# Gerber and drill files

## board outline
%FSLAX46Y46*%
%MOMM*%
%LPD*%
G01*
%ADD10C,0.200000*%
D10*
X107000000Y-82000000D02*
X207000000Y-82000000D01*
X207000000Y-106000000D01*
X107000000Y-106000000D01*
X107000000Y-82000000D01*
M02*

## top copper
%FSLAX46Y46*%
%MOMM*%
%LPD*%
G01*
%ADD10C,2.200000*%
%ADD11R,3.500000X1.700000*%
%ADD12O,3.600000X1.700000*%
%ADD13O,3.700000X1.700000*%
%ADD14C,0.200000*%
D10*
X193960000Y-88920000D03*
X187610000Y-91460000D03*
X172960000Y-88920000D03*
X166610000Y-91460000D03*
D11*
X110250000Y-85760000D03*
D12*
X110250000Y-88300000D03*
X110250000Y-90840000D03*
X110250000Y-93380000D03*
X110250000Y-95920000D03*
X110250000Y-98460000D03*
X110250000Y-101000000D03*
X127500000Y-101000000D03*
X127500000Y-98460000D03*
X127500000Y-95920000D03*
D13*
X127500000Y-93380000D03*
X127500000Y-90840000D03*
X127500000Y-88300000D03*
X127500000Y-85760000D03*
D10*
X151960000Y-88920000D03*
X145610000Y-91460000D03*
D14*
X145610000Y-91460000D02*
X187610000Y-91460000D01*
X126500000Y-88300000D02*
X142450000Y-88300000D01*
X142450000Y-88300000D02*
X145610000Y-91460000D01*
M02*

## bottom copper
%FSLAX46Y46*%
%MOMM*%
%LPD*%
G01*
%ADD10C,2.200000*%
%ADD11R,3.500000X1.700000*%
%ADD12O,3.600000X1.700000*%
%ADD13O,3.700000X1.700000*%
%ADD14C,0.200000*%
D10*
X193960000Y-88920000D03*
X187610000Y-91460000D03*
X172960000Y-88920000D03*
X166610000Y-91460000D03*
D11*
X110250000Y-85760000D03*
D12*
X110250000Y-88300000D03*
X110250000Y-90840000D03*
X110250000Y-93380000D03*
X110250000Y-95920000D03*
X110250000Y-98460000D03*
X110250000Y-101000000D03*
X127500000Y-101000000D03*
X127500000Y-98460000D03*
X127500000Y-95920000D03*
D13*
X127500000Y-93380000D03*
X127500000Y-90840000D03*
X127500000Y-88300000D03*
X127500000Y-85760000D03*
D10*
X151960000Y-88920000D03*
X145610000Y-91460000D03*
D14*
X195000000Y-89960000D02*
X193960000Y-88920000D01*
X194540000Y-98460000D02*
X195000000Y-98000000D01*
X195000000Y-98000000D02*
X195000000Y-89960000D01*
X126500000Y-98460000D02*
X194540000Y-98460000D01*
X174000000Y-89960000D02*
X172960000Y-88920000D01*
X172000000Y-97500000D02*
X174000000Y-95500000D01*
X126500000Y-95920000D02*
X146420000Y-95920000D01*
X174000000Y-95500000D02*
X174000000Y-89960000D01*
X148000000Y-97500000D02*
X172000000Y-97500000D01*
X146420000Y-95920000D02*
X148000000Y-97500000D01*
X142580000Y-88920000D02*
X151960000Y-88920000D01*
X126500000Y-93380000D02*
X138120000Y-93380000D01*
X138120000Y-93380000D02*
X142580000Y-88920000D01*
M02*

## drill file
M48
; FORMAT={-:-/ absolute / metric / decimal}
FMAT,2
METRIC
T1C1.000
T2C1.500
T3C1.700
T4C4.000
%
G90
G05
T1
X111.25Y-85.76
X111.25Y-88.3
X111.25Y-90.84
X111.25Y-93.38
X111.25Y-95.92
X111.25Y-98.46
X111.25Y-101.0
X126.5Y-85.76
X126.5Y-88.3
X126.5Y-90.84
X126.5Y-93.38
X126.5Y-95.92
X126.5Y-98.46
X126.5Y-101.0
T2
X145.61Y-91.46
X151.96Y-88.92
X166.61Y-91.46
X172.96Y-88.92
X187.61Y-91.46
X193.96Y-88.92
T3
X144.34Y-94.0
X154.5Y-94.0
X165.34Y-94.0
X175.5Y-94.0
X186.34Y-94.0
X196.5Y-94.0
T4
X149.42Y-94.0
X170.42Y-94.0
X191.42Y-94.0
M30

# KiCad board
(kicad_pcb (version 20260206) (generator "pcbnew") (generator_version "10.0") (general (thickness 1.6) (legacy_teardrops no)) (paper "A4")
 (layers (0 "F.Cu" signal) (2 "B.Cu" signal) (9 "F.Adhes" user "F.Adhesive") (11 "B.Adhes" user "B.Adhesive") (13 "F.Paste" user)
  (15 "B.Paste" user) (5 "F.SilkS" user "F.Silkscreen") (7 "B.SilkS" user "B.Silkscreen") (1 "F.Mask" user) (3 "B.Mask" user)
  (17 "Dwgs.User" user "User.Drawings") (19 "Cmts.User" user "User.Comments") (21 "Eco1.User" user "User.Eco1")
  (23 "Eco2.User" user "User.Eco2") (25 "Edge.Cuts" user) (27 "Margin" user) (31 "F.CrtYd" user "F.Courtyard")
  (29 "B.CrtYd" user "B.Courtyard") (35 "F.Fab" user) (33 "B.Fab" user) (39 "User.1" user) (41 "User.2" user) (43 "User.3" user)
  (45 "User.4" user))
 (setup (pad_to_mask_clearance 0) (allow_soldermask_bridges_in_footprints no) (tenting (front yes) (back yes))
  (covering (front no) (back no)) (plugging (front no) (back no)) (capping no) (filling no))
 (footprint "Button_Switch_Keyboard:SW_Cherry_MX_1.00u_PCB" (layer "F.Cu") (at 193.96 88.92)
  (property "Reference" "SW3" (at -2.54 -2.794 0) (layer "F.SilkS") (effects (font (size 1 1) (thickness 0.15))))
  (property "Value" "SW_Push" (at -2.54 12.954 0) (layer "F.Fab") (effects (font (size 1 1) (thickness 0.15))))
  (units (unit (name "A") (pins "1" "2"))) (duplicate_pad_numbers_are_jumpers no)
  (pad "" np_thru_hole circle (at -7.62 5.08) (size 1.7 1.7) (drill 1.7) (layers "*.Cu" "*.Mask"))
  (pad "" np_thru_hole circle (at -2.54 5.08) (size 4 4) (drill 4) (layers "*.Cu" "*.Mask"))
  (pad "" np_thru_hole circle (at 2.54 5.08) (size 1.7 1.7) (drill 1.7) (layers "*.Cu" "*.Mask"))
  (pad "1" thru_hole circle (at 0 0) (size 2.2 2.2) (drill 1.5) (layers "*.Cu" "*.Mask") (remove_unused_layers no)
   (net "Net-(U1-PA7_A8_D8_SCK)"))
  (pad "2" thru_hole circle (at -6.35 2.54) (size 2.2 2.2) (drill 1.5) (layers "*.Cu" "*.Mask") (remove_unused_layers no) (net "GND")))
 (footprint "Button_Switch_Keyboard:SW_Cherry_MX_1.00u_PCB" (layer "F.Cu") (at 172.96 88.92)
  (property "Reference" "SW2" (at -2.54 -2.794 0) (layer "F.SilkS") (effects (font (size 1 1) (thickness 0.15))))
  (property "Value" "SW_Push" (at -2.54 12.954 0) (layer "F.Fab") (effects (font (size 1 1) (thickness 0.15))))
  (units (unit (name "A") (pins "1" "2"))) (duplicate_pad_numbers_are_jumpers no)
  (pad "" np_thru_hole circle (at -7.62 5.08) (size 1.7 1.7) (drill 1.7) (layers "*.Cu" "*.Mask"))
  (pad "" np_thru_hole circle (at -2.54 5.08) (size 4 4) (drill 4) (layers "*.Cu" "*.Mask"))
  (pad "" np_thru_hole circle (at 2.54 5.08) (size 1.7 1.7) (drill 1.7) (layers "*.Cu" "*.Mask"))
  (pad "1" thru_hole circle (at 0 0) (size 2.2 2.2) (drill 1.5) (layers "*.Cu" "*.Mask") (remove_unused_layers no)
   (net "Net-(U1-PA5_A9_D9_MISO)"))
  (pad "2" thru_hole circle (at -6.35 2.54) (size 2.2 2.2) (drill 1.5) (layers "*.Cu" "*.Mask") (remove_unused_layers no) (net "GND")))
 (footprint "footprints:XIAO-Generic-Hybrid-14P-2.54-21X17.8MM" (layer "F.Cu") (at 118.875 93.38)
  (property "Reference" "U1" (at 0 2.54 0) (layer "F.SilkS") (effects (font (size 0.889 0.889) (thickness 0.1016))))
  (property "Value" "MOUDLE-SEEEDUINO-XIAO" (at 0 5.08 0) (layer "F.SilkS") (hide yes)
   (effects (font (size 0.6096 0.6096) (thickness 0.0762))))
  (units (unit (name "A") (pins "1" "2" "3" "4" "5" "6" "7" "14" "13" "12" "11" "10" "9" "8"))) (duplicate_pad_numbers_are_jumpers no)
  (pad "1" thru_hole rect (at -7.625 -7.62) (size 3.5 1.7) (drill 1 (offset -1 0)) (layers "*.Cu" "*.Mask") (remove_unused_layers no)
   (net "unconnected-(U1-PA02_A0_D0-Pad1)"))
  (pad "2" thru_hole oval (at -7.625 -5.08) (size 3.6 1.7) (drill 1 (offset -1 0)) (layers "*.Cu" "*.Mask") (remove_unused_layers no)
   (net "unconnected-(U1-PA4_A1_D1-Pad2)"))
  (pad "3" thru_hole oval (at -7.625 -2.54) (size 3.6 1.7) (drill 1 (offset -1 0)) (layers "*.Cu" "*.Mask") (remove_unused_layers no)
   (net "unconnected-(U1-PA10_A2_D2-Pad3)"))
  (pad "4" thru_hole oval (at -7.625 0) (size 3.6 1.7) (drill 1 (offset -1 0)) (layers "*.Cu" "*.Mask") (remove_unused_layers no)
   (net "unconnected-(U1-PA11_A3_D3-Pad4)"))
  (pad "5" thru_hole oval (at -7.625 2.54) (size 3.6 1.7) (drill 1 (offset -1 0)) (layers "*.Cu" "*.Mask") (remove_unused_layers no)
   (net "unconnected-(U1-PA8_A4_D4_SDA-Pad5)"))
  (pad "6" thru_hole oval (at -7.625 5.08 180) (size 3.6 1.7) (drill 1 (offset 1 0)) (layers "*.Cu" "*.Mask") (remove_unused_layers no)
   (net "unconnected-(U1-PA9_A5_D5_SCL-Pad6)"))
  (pad "7" thru_hole oval (at -7.625 7.62) (size 3.6 1.7) (drill 1 (offset -1 0)) (layers "*.Cu" "*.Mask") (remove_unused_layers no)
   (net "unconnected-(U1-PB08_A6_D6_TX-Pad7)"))
  (pad "8" thru_hole oval (at 7.625 7.62) (size 3.6 1.7) (drill 1 (offset 1 0)) (layers "*.Cu" "*.Mask") (remove_unused_layers no)
   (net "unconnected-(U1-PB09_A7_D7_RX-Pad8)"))
  (pad "9" thru_hole oval (at 7.625 5.08) (size 3.6 1.7) (drill 1 (offset 1 0)) (layers "*.Cu" "*.Mask") (remove_unused_layers no)
   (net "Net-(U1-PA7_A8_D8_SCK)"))
  (pad "10" thru_hole oval (at 7.625 2.54) (size 3.6 1.7) (drill 1 (offset 1 0)) (layers "*.Cu" "*.Mask") (remove_unused_layers no)
   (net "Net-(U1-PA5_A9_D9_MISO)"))
  (pad "11" thru_hole oval (at 7.625 0) (size 3.7 1.7) (drill 1 (offset 1 0)) (layers "*.Cu" "*.Mask") (remove_unused_layers no)
   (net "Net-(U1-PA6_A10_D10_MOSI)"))
  (pad "12" thru_hole oval (at 7.625 -2.54) (size 3.7 1.7) (drill 1 (offset 1 0)) (layers "*.Cu" "*.Mask") (remove_unused_layers no)
   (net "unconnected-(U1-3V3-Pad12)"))
  (pad "13" thru_hole oval (at 7.625 -5.08) (size 3.7 1.7) (drill 1 (offset 1 0)) (layers "*.Cu" "*.Mask") (remove_unused_layers no)
   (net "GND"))
  (pad "14" thru_hole oval (at 7.625 -7.62) (size 3.7 1.7) (drill 1 (offset 1 0)) (layers "*.Cu" "*.Mask") (remove_unused_layers no)
   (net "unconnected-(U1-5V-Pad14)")))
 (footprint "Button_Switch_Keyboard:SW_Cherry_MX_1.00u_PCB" (layer "F.Cu") (at 151.96 88.92)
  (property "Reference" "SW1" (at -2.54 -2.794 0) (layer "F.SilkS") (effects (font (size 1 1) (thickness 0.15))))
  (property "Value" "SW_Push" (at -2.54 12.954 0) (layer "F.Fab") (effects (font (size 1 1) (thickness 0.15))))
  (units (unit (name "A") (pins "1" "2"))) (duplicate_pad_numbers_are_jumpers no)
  (pad "" np_thru_hole circle (at -7.62 5.08) (size 1.7 1.7) (drill 1.7) (layers "*.Cu" "*.Mask"))
  (pad "" np_thru_hole circle (at -2.54 5.08) (size 4 4) (drill 4) (layers "*.Cu" "*.Mask"))
  (pad "" np_thru_hole circle (at 2.54 5.08) (size 1.7 1.7) (drill 1.7) (layers "*.Cu" "*.Mask"))
  (pad "1" thru_hole circle (at 0 0) (size 2.2 2.2) (drill 1.5) (layers "*.Cu" "*.Mask") (remove_unused_layers no)
   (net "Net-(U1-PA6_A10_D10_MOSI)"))
  (pad "2" thru_hole circle (at -6.35 2.54) (size 2.2 2.2) (drill 1.5) (layers "*.Cu" "*.Mask") (remove_unused_layers no) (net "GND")))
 (gr_rect (start 107 82) (end 207 106) (stroke (width 0.2) (type default)) (fill no) (layer "Edge.Cuts"))
 (segment (start 195 89.96) (end 193.96 88.92) (width 0.2) (layer "B.Cu") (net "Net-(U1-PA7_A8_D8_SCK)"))
 (segment (start 194.54 98.46) (end 195 98) (width 0.2) (layer "B.Cu") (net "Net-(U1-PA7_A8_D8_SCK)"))
 (segment (start 195 98) (end 195 89.96) (width 0.2) (layer "B.Cu") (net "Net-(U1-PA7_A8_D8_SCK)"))
 (segment (start 126.5 98.46) (end 194.54 98.46) (width 0.2) (layer "B.Cu") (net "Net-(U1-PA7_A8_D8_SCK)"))
 (segment (start 145.61 91.46) (end 187.61 91.46) (width 0.2) (layer "F.Cu") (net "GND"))
 (segment (start 126.5 88.3) (end 142.45 88.3) (width 0.2) (layer "F.Cu") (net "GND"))
 (segment (start 142.45 88.3) (end 145.61 91.46) (width 0.2) (layer "F.Cu") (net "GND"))
 (segment (start 174 89.96) (end 172.96 88.92) (width 0.2) (layer "B.Cu") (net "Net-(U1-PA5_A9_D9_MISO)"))
 (segment (start 172 97.5) (end 174 95.5) (width 0.2) (layer "B.Cu") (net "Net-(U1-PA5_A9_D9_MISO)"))
 (segment (start 126.5 95.92) (end 146.42 95.92) (width 0.2) (layer "B.Cu") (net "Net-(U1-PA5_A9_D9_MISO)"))
 (segment (start 174 95.5) (end 174 89.96) (width 0.2) (layer "B.Cu") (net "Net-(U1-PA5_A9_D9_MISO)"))
 (segment (start 148 97.5) (end 172 97.5) (width 0.2) (layer "B.Cu") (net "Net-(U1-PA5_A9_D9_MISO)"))
 (segment (start 146.42 95.92) (end 148 97.5) (width 0.2) (layer "B.Cu") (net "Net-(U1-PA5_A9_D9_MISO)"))
 (segment (start 142.58 88.92) (end 151.96 88.92) (width 0.2) (layer "B.Cu") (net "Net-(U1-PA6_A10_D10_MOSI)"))
 (segment (start 126.5 93.38) (end 138.12 93.38) (width 0.2) (layer "B.Cu") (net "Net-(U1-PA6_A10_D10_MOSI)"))
 (segment (start 138.12 93.38) (end 142.58 88.92) (width 0.2) (layer "B.Cu") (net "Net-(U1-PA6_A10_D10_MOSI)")))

